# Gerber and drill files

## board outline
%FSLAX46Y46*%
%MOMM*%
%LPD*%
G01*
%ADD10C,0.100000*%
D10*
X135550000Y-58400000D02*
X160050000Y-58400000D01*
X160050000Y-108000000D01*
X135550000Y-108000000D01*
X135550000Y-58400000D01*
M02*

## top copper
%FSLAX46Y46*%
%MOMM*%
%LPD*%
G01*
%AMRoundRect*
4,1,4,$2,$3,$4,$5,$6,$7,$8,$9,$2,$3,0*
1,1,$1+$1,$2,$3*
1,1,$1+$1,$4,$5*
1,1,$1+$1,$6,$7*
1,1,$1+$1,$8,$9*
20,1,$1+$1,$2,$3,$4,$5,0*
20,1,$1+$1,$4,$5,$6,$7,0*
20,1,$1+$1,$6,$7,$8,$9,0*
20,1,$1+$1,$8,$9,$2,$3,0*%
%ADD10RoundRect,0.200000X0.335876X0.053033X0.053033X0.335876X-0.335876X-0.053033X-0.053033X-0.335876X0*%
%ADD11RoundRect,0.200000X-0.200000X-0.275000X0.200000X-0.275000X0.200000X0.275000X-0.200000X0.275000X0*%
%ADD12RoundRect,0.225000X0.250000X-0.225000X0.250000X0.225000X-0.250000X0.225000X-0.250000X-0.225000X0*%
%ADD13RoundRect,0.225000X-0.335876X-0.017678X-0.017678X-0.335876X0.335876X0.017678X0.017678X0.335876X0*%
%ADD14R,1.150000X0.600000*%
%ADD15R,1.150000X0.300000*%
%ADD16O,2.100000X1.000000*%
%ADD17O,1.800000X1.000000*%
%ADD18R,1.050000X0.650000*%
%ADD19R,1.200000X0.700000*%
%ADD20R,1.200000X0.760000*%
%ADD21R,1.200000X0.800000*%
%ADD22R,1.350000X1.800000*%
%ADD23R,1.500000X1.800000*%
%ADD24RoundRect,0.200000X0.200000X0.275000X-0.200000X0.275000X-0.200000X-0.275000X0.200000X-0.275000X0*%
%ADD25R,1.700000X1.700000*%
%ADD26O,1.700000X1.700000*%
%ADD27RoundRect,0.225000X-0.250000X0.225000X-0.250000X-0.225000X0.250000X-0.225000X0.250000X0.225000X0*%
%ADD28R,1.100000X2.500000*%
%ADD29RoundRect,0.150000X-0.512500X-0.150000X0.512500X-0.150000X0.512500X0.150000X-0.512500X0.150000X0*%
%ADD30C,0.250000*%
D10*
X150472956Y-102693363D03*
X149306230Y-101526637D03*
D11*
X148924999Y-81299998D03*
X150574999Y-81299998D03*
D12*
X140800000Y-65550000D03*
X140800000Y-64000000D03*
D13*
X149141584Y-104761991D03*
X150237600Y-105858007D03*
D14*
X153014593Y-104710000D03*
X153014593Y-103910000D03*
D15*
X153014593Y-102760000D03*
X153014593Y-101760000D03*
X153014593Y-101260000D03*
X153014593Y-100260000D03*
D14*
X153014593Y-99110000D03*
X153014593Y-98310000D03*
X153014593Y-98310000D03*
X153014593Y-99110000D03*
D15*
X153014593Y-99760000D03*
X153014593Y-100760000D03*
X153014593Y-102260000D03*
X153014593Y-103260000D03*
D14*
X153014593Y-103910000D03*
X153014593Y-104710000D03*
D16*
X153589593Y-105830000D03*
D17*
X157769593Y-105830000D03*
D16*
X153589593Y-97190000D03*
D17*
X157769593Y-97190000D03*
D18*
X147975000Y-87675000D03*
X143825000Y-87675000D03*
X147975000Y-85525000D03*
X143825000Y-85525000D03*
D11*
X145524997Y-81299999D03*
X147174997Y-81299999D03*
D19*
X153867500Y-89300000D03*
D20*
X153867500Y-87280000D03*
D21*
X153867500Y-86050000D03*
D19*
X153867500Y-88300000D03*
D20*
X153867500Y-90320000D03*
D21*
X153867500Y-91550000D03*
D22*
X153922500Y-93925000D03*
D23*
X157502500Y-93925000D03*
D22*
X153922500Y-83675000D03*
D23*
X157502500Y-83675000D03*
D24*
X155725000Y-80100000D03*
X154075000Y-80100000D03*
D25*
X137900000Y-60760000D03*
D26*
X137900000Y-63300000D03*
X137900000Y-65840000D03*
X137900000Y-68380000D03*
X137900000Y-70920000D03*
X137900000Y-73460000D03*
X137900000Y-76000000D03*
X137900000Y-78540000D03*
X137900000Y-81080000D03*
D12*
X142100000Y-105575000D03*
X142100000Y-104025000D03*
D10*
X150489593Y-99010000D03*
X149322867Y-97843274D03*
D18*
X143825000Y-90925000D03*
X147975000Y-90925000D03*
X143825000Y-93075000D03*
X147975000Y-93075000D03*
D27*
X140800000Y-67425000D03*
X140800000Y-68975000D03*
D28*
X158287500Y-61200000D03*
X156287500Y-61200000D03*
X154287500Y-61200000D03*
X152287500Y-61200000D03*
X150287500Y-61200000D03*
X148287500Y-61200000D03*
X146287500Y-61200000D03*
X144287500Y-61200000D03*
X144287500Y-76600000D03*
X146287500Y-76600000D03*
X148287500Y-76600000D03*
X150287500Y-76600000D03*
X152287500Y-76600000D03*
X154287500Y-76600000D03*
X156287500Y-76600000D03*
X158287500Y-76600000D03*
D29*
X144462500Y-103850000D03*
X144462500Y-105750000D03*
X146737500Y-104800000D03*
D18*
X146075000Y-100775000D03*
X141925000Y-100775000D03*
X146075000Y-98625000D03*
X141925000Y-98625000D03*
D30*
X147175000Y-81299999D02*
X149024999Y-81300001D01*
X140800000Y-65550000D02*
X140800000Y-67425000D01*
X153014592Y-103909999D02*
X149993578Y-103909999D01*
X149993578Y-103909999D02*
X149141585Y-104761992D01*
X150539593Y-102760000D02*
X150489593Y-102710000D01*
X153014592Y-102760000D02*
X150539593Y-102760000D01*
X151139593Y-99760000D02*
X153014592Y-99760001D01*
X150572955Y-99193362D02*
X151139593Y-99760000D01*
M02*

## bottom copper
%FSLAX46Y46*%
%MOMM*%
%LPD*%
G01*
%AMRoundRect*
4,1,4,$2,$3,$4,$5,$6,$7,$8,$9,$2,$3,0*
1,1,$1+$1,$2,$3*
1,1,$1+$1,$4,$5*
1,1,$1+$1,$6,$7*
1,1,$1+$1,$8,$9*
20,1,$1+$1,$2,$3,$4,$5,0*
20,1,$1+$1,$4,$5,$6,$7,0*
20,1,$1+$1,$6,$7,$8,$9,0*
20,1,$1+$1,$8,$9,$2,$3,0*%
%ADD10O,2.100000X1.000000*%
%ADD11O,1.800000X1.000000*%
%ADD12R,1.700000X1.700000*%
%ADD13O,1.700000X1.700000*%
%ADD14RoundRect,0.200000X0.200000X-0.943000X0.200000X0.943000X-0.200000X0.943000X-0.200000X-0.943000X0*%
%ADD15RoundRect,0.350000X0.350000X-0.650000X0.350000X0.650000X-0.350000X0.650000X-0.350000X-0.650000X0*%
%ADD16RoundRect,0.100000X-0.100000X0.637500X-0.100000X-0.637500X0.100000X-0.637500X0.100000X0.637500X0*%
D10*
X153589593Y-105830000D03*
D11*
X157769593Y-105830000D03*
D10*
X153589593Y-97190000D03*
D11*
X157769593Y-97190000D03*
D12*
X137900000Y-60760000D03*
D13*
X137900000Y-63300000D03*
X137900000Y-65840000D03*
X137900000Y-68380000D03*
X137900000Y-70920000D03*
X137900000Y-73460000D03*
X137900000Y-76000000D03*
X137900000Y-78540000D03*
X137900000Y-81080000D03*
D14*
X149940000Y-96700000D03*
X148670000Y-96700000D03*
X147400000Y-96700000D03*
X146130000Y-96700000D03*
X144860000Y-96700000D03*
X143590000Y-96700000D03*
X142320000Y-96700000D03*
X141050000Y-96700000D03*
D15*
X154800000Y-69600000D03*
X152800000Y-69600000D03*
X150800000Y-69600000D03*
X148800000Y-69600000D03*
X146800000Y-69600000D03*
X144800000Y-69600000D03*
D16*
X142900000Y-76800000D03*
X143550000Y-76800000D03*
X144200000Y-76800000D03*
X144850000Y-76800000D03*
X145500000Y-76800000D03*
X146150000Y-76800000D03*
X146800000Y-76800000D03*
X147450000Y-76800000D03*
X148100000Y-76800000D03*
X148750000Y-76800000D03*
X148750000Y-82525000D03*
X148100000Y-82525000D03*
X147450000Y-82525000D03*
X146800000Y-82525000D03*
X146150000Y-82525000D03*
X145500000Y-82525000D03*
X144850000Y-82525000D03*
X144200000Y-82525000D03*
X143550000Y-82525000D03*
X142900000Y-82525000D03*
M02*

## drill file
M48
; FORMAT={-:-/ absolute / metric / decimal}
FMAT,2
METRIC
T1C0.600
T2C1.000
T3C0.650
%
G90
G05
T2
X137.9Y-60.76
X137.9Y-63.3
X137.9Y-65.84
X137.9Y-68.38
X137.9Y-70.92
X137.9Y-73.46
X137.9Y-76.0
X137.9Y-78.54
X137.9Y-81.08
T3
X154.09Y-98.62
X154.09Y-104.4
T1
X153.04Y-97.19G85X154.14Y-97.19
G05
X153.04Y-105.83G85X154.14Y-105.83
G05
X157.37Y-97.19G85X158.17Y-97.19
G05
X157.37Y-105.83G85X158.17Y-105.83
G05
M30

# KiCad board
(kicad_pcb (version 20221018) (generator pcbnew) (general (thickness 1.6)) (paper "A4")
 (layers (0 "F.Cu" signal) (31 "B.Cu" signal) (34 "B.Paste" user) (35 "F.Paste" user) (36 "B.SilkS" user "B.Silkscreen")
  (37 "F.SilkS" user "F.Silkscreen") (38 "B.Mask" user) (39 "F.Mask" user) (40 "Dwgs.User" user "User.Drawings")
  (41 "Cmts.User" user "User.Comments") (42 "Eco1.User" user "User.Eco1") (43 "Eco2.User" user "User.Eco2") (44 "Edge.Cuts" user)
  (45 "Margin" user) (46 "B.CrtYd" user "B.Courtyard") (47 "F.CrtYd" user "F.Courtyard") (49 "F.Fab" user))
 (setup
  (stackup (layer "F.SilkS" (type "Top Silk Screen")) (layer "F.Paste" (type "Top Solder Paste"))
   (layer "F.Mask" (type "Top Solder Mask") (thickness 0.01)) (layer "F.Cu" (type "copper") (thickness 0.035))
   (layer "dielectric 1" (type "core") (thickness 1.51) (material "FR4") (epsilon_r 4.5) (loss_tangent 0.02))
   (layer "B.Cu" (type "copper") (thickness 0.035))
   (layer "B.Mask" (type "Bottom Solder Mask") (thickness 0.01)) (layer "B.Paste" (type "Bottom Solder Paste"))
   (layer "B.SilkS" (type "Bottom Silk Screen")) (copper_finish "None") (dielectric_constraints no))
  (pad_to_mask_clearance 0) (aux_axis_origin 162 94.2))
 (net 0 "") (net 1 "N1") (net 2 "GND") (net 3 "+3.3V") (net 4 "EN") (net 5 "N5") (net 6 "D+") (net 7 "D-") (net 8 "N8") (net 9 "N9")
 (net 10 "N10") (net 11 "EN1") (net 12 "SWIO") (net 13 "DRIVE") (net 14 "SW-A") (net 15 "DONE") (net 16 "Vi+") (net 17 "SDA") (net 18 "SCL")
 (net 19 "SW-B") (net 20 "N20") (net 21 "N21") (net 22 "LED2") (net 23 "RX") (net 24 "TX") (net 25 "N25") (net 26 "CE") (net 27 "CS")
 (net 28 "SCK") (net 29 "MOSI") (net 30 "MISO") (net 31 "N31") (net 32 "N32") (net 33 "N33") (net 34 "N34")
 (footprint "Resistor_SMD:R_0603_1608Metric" (layer "F.Cu") (at 149.889593 102.11 135)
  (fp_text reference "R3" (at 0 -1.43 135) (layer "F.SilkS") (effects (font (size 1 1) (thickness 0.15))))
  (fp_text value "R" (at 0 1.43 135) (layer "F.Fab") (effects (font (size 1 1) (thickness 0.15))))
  (pad "1" smd roundrect (at -0.825 0 135) (size 0.8 0.95) (layers "F.Cu" "F.Paste" "F.Mask") (roundrect_rratio 0.25) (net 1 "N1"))
  (pad "2" smd roundrect (at 0.825 0 135) (size 0.8 0.95) (layers "F.Cu" "F.Paste" "F.Mask") (roundrect_rratio 0.25) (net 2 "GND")))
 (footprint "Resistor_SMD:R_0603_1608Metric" (layer "F.Cu") (at 149.749999 81.299998)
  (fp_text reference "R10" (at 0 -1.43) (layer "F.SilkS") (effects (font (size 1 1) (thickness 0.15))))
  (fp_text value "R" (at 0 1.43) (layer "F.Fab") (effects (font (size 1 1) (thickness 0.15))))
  (pad "1" smd roundrect (at -0.825 0) (size 0.8 0.95) (layers "F.Cu" "F.Paste" "F.Mask") (roundrect_rratio 0.25) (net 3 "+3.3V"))
  (pad "2" smd roundrect (at 0.825 0) (size 0.8 0.95) (layers "F.Cu" "F.Paste" "F.Mask") (roundrect_rratio 0.25) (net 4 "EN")))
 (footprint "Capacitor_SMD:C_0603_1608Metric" (layer "F.Cu") (at 140.8 64.775 90)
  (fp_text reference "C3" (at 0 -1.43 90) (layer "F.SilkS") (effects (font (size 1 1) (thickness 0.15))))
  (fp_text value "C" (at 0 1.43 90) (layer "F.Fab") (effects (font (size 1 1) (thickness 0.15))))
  (pad "1" smd roundrect (at -0.775 0 90) (size 0.9 0.95) (layers "F.Cu" "F.Paste" "F.Mask") (roundrect_rratio 0.25) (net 3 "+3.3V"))
  (pad "2" smd roundrect (at 0.775 0 90) (size 0.9 0.95) (layers "F.Cu" "F.Paste" "F.Mask") (roundrect_rratio 0.25) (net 2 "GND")))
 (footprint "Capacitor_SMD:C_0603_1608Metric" (layer "F.Cu") (at 149.689592 105.309999 -45)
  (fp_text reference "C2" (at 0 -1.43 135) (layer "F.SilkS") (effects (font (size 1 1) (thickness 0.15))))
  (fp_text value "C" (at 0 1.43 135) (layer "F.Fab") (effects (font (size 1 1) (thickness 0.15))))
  (pad "1" smd roundrect (at -0.775 0 315) (size 0.9 0.95) (layers "F.Cu" "F.Paste" "F.Mask") (roundrect_rratio 0.25) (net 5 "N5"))
  (pad "2" smd roundrect (at 0.775 0 315) (size 0.9 0.95) (layers "F.Cu" "F.Paste" "F.Mask") (roundrect_rratio 0.25) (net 2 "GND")))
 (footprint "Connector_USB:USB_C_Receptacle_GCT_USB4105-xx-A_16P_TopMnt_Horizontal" (layer "F.Cu") (at 156.694593 101.51 90)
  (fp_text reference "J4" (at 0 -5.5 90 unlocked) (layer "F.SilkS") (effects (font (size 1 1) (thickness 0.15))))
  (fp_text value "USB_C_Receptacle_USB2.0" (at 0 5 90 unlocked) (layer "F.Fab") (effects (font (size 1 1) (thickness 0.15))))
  (pad "" np_thru_hole circle (at -2.89 -2.605 90) (size 0.65 0.65) (drill 0.65) (layers "F&B.Cu" "*.Mask"))
  (pad "" np_thru_hole circle (at 2.89 -2.605 90) (size 0.65 0.65) (drill 0.65) (layers "F&B.Cu" "*.Mask"))
  (pad "A1" smd rect (at -3.2 -3.68 90) (size 0.6 1.15) (layers "F.Cu" "F.Paste" "F.Mask") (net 2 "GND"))
  (pad "A4" smd rect (at -2.4 -3.68 90) (size 0.6 1.15) (layers "F.Cu" "F.Paste" "F.Mask") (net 5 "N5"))
  (pad "A5" smd rect (at -1.25 -3.68 90) (size 0.3 1.15) (layers "F.Cu" "F.Paste" "F.Mask") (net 1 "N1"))
  (pad "A6" smd rect (at -0.25 -3.68 90) (size 0.3 1.15) (layers "F.Cu" "F.Paste" "F.Mask") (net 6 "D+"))
  (pad "A7" smd rect (at 0.25 -3.68 90) (size 0.3 1.15) (layers "F.Cu" "F.Paste" "F.Mask") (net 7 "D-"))
  (pad "A8" smd rect (at 1.25 -3.68 90) (size 0.3 1.15) (layers "F.Cu" "F.Paste" "F.Mask") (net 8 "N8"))
  (pad "A9" smd rect (at 2.4 -3.68 90) (size 0.6 1.15) (layers "F.Cu" "F.Paste" "F.Mask") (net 5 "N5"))
  (pad "A12" smd rect (at 3.2 -3.68 90) (size 0.6 1.15) (layers "F.Cu" "F.Paste" "F.Mask") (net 2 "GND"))
  (pad "B1" smd rect (at 3.2 -3.68 90) (size 0.6 1.15) (layers "F.Cu" "F.Paste" "F.Mask") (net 2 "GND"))
  (pad "B4" smd rect (at 2.4 -3.68 90) (size 0.6 1.15) (layers "F.Cu" "F.Paste" "F.Mask") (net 5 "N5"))
  (pad "B5" smd rect (at 1.75 -3.68 90) (size 0.3 1.15) (layers "F.Cu" "F.Paste" "F.Mask") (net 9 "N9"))
  (pad "B6" smd rect (at 0.75 -3.68 90) (size 0.3 1.15) (layers "F.Cu" "F.Paste" "F.Mask") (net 6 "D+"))
  (pad "B7" smd rect (at -0.75 -3.68 90) (size 0.3 1.15) (layers "F.Cu" "F.Paste" "F.Mask") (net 7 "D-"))
  (pad "B8" smd rect (at -1.75 -3.68 90) (size 0.3 1.15) (layers "F.Cu" "F.Paste" "F.Mask") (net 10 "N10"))
  (pad "B9" smd rect (at -2.4 -3.68 90) (size 0.6 1.15) (layers "F.Cu" "F.Paste" "F.Mask") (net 5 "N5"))
  (pad "B12" smd rect (at -3.2 -3.68 90) (size 0.6 1.15) (layers "F.Cu" "F.Paste" "F.Mask") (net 2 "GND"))
  (pad "S1" thru_hole oval (at -4.32 -3.105 90) (size 1 2.1) (drill oval 0.6 1.7) (layers "*.Cu" "*.Mask" "F.Paste") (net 2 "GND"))
  (pad "S1" thru_hole oval (at -4.32 1.075 90) (size 1 1.8) (drill oval 0.6 1.4) (layers "*.Cu" "*.Mask" "F.Paste") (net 2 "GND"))
  (pad "S1" thru_hole oval (at 4.32 -3.105 90) (size 1 2.1) (drill oval 0.6 1.7) (layers "*.Cu" "*.Mask" "F.Paste") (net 2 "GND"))
  (pad "S1" thru_hole oval (at 4.32 1.075 90) (size 1 1.8) (drill oval 0.6 1.4) (layers "*.Cu" "*.Mask" "F.Paste") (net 2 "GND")))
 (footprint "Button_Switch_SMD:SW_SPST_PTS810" (layer "F.Cu") (at 145.9 86.6 180)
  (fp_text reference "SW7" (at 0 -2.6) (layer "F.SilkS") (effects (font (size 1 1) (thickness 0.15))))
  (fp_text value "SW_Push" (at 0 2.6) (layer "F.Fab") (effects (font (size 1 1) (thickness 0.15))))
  (pad "1" smd rect (at -2.075 -1.075 180) (size 1.05 0.65) (layers "F.Cu" "F.Paste" "F.Mask") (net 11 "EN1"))
  (pad "1" smd rect (at 2.075 -1.075 180) (size 1.05 0.65) (layers "F.Cu" "F.Paste" "F.Mask") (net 11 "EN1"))
  (pad "2" smd rect (at -2.075 1.075 180) (size 1.05 0.65) (layers "F.Cu" "F.Paste" "F.Mask") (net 2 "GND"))
  (pad "2" smd rect (at 2.075 1.075 180) (size 1.05 0.65) (layers "F.Cu" "F.Paste" "F.Mask") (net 2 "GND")))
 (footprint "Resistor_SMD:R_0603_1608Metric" (layer "F.Cu") (at 146.349997 81.299999)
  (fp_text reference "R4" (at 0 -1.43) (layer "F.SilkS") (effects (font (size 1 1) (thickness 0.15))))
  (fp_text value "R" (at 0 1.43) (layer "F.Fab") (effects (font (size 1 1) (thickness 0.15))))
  (pad "1" smd roundrect (at -0.825 0) (size 0.8 0.95) (layers "F.Cu" "F.Paste" "F.Mask") (roundrect_rratio 0.25) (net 11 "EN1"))
  (pad "2" smd roundrect (at 0.825 0) (size 0.8 0.95) (layers "F.Cu" "F.Paste" "F.Mask") (roundrect_rratio 0.25) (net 3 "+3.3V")))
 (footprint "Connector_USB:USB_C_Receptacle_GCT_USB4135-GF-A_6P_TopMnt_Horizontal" (layer "F.Cu") (at 156.9 88.8 90)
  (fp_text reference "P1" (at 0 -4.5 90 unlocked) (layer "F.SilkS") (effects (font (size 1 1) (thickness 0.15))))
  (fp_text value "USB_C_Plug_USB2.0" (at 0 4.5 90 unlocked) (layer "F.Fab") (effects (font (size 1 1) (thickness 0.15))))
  (pad "A5" smd rect (at -0.5 -3.0325 90) (size 0.7 1.2) (layers "F.Cu" "F.Paste" "F.Mask") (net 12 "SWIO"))
  (pad "A9" smd rect (at 1.52 -3.0325 270) (size 0.76 1.2) (layers "F.Cu" "F.Paste" "F.Mask") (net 3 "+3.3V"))
  (pad "A12" smd rect (at 2.75 -3.0325 270) (size 0.8 1.2) (layers "F.Cu" "F.Paste" "F.Mask") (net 2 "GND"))
  (pad "B5" smd rect (at 0.5 -3.0325 270) (size 0.7 1.2) (layers "F.Cu" "F.Paste" "F.Mask") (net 12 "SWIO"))
  (pad "B9" smd rect (at -1.52 -3.0325 90) (size 0.76 1.2) (layers "F.Cu" "F.Paste" "F.Mask") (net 3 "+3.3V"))
  (pad "B12" smd rect (at -2.75 -3.0325 90) (size 0.8 1.2) (layers "F.Cu" "F.Paste" "F.Mask") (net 2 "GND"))
  (pad "S1" smd rect (at -5.125 -2.9775 90) (size 1.8 1.35) (layers "F.Cu" "F.Paste" "F.Mask") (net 2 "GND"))
  (pad "S1" smd rect (at -5.125 0.6025 90) (size 1.8 1.5) (layers "F.Cu" "F.Paste" "F.Mask") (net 2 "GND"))
  (pad "S1" smd rect (at 5.125 -2.9775 90) (size 1.8 1.35) (layers "F.Cu" "F.Paste" "F.Mask") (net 2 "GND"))
  (pad "S1" smd rect (at 5.125 0.6025 90) (size 1.8 1.5) (layers "F.Cu" "F.Paste" "F.Mask") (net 2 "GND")))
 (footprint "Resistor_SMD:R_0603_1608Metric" (layer "F.Cu") (at 154.9 80.1 180)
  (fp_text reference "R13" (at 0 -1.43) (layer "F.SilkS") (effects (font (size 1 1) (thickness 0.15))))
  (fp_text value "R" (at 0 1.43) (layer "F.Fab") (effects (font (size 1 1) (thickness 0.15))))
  (pad "1" smd roundrect (at -0.825 0 180) (size 0.8 0.95) (layers "F.Cu" "F.Paste" "F.Mask") (roundrect_rratio 0.25) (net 2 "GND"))
  (pad "2" smd roundrect (at 0.825 0 180) (size 0.8 0.95) (layers "F.Cu" "F.Paste" "F.Mask") (roundrect_rratio 0.25) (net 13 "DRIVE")))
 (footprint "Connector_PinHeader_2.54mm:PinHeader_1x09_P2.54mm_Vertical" (layer "F.Cu") (at 137.9 60.76)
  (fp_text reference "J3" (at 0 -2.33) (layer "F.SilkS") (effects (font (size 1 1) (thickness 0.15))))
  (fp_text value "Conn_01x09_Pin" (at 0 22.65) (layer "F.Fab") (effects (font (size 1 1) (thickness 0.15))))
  (pad "1" thru_hole rect (at 0 0) (size 1.7 1.7) (drill 1) (layers "*.Cu" "*.Mask") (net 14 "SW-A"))
  (pad "2" thru_hole oval (at 0 2.54) (size 1.7 1.7) (drill 1) (layers "*.Cu" "*.Mask") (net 2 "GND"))
  (pad "3" thru_hole oval (at 0 5.08) (size 1.7 1.7) (drill 1) (layers "*.Cu" "*.Mask") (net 3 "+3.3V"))
  (pad "4" thru_hole oval (at 0 7.62) (size 1.7 1.7) (drill 1) (layers "*.Cu" "*.Mask") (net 13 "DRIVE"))
  (pad "5" thru_hole oval (at 0 10.16) (size 1.7 1.7) (drill 1) (layers "*.Cu" "*.Mask") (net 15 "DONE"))
  (pad "6" thru_hole oval (at 0 12.7) (size 1.7 1.7) (drill 1) (layers "*.Cu" "*.Mask") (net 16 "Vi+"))
  (pad "7" thru_hole oval (at 0 15.24) (size 1.7 1.7) (drill 1) (layers "*.Cu" "*.Mask") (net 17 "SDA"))
  (pad "8" thru_hole oval (at 0 17.78) (size 1.7 1.7) (drill 1) (layers "*.Cu" "*.Mask") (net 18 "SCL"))
  (pad "9" thru_hole oval (at 0 20.32) (size 1.7 1.7) (drill 1) (layers "*.Cu" "*.Mask") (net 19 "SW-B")))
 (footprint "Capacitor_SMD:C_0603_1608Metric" (layer "F.Cu") (at 142.1 104.8 90)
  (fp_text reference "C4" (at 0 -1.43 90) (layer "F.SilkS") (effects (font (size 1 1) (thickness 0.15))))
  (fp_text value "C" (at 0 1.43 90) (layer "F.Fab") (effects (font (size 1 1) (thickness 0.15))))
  (pad "1" smd roundrect (at -0.775 0 90) (size 0.9 0.95) (layers "F.Cu" "F.Paste" "F.Mask") (roundrect_rratio 0.25) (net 3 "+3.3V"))
  (pad "2" smd roundrect (at 0.775 0 90) (size 0.9 0.95) (layers "F.Cu" "F.Paste" "F.Mask") (roundrect_rratio 0.25) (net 2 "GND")))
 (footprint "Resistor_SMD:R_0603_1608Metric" (layer "F.Cu") (at 149.90623 98.426637 135)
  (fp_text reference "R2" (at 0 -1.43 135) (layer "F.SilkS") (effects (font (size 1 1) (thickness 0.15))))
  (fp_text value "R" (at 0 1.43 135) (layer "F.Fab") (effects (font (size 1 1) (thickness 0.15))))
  (pad "1" smd roundrect (at -0.825 0 135) (size 0.8 0.95) (layers "F.Cu" "F.Paste" "F.Mask") (roundrect_rratio 0.25) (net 9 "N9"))
  (pad "2" smd roundrect (at 0.825 0 135) (size 0.8 0.95) (layers "F.Cu" "F.Paste" "F.Mask") (roundrect_rratio 0.25) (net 2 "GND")))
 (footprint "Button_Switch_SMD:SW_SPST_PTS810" (layer "F.Cu") (at 145.9 92)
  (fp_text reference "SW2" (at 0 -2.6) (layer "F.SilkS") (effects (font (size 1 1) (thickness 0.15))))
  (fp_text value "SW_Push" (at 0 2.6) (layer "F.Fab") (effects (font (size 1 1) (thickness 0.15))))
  (pad "1" smd rect (at -2.075 -1.075) (size 1.05 0.65) (layers "F.Cu" "F.Paste" "F.Mask") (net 2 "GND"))
  (pad "1" smd rect (at 2.075 -1.075) (size 1.05 0.65) (layers "F.Cu" "F.Paste" "F.Mask") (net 2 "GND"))
  (pad "2" smd rect (at -2.075 1.075) (size 1.05 0.65) (layers "F.Cu" "F.Paste" "F.Mask") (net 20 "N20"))
  (pad "2" smd rect (at 2.075 1.075) (size 1.05 0.65) (layers "F.Cu" "F.Paste" "F.Mask") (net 20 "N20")))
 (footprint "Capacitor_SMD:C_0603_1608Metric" (layer "F.Cu") (at 140.8 68.2 -90)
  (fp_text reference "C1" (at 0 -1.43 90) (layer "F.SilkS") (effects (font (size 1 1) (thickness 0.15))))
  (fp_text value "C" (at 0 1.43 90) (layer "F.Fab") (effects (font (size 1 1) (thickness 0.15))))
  (pad "1" smd roundrect (at -0.775 0 270) (size 0.9 0.95) (layers "F.Cu" "F.Paste" "F.Mask") (roundrect_rratio 0.25) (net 3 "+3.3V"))
  (pad "2" smd roundrect (at 0.775 0 270) (size 0.9 0.95) (layers "F.Cu" "F.Paste" "F.Mask") (roundrect_rratio 0.25) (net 2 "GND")))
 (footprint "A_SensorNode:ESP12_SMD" (layer "F.Cu") (at 160.8875 60.85 -90)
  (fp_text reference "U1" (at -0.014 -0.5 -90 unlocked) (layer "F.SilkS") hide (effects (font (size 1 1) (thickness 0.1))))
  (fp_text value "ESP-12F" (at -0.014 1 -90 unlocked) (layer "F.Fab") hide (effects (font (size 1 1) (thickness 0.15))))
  (pad "1" smd rect (at 1.05 2.6 270) (size 2.5 1.1) (drill (offset -0.7 0)) (layers "F.Cu" "F.Paste" "F.Mask") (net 11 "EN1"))
  (pad "2" smd rect (at 1.05 4.6 270) (size 2.5 1.1) (drill (offset -0.7 0)) (layers "F.Cu" "F.Paste" "F.Mask") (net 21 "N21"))
  (pad "3" smd rect (at 1.05 6.6 270) (size 2.5 1.1) (drill (offset -0.7 0)) (layers "F.Cu" "F.Paste" "F.Mask") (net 4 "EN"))
  (pad "4" smd rect (at 1.05 8.6 270) (size 2.5 1.1) (drill (offset -0.7 0)) (layers "F.Cu" "F.Paste" "F.Mask") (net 11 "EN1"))
  (pad "5" smd rect (at 1.05 10.6 270) (size 2.5 1.1) (drill (offset -0.7 0)) (layers "F.Cu" "F.Paste" "F.Mask") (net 14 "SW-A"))
  (pad "6" smd rect (at 1.05 12.6 270) (size 2.5 1.1) (drill (offset -0.7 0)) (layers "F.Cu" "F.Paste" "F.Mask") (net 19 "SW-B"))
  (pad "7" smd rect (at 1.05 14.6 270) (size 2.5 1.1) (drill (offset -0.7 0)) (layers "F.Cu" "F.Paste" "F.Mask") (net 15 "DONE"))
  (pad "8" smd rect (at 1.05 16.6 270) (size 2.5 1.1) (drill (offset -0.7 0)) (layers "F.Cu" "F.Paste" "F.Mask") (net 3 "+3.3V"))
  (pad "9" smd rect (at 15.05 16.6 270) (size 2.5 1.1) (drill (offset 0.7 0)) (layers "F.Cu" "F.Paste" "F.Mask") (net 2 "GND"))
  (pad "10" smd rect (at 15.05 14.6 270) (size 2.5 1.1) (drill (offset 0.7 0)) (layers "F.Cu" "F.Paste" "F.Mask") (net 13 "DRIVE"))
  (pad "11" smd rect (at 15.05 12.6 270) (size 2.5 1.1) (drill (offset 0.7 0)) (layers "F.Cu" "F.Paste" "F.Mask") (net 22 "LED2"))
  (pad "12" smd rect (at 15.05 10.6 270) (size 2.5 1.1) (drill (offset 0.7 0)) (layers "F.Cu" "F.Paste" "F.Mask") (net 20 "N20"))
  (pad "13" smd rect (at 15.05 8.6 270) (size 2.5 1.1) (drill (offset 0.7 0)) (layers "F.Cu" "F.Paste" "F.Mask") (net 17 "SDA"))
  (pad "14" smd rect (at 15.05 6.6 270) (size 2.5 1.1) (drill (offset 0.7 0)) (layers "F.Cu" "F.Paste" "F.Mask") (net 18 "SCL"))
  (pad "15" smd rect (at 15.05 4.6 270) (size 2.5 1.1) (drill (offset 0.7 0)) (layers "F.Cu" "F.Paste" "F.Mask") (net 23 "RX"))
  (pad "16" smd rect (at 15.05 2.6 270) (size 2.5 1.1) (drill (offset 0.7 0)) (layers "F.Cu" "F.Paste" "F.Mask") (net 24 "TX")))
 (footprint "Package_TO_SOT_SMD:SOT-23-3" (layer "F.Cu") (at 145.6 104.8)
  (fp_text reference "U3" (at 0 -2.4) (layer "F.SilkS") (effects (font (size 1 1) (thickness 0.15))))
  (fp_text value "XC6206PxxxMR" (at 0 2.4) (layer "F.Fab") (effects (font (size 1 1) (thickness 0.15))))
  (pad "1" smd roundrect (at -1.1375 -0.95) (size 1.325 0.6) (layers "F.Cu" "F.Paste" "F.Mask") (roundrect_rratio 0.25) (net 2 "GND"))
  (pad "2" smd roundrect (at -1.1375 0.95) (size 1.325 0.6) (layers "F.Cu" "F.Paste" "F.Mask") (roundrect_rratio 0.25) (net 3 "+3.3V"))
  (pad "3" smd roundrect (at 1.1375 0) (size 1.325 0.6) (layers "F.Cu" "F.Paste" "F.Mask") (roundrect_rratio 0.25) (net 5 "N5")))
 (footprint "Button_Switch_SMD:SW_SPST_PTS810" (layer "F.Cu") (at 144 99.7 180)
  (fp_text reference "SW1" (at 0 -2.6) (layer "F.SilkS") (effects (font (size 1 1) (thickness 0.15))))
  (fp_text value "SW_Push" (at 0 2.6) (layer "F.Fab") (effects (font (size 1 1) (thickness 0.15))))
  (pad "1" smd rect (at -2.075 -1.075 180) (size 1.05 0.65) (layers "F.Cu" "F.Paste" "F.Mask") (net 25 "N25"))
  (pad "1" smd rect (at 2.075 -1.075 180) (size 1.05 0.65) (layers "F.Cu" "F.Paste" "F.Mask") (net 25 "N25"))
  (pad "2" smd rect (at -2.075 1.075 180) (size 1.05 0.65) (layers "F.Cu" "F.Paste" "F.Mask") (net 2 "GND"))
  (pad "2" smd rect (at 2.075 1.075 180) (size 1.05 0.65) (layers "F.Cu" "F.Paste" "F.Mask") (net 2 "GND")))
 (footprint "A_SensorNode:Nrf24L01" (layer "B.Cu") (at 149.94 96.7 90)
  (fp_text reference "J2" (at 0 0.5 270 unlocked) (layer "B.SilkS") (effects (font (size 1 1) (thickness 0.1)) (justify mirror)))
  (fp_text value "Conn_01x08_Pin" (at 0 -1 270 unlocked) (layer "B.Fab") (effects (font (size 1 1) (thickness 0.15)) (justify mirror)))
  (pad "1" smd roundrect (at 0 0 90) (size 2.286 0.8) (layers "B.Cu" "B.Paste" "B.Mask") (roundrect_rratio 0.25) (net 3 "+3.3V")
   (thermal_bridge_angle 45))
  (pad "2" smd roundrect (at 0 -1.27 90) (size 2.286 0.8) (layers "B.Cu" "B.Paste" "B.Mask") (roundrect_rratio 0.25) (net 2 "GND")
   (thermal_bridge_angle 45))
  (pad "3" smd roundrect (at 0 -2.54 90) (size 2.286 0.8) (layers "B.Cu" "B.Paste" "B.Mask") (roundrect_rratio 0.25) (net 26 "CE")
   (thermal_bridge_angle 45))
  (pad "4" smd roundrect (at 0 -3.81 90) (size 2.286 0.8) (layers "B.Cu" "B.Paste" "B.Mask") (roundrect_rratio 0.25) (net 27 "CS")
   (thermal_bridge_angle 45))
  (pad "5" smd roundrect (at 0 -5.08 90) (size 2.286 0.8) (layers "B.Cu" "B.Paste" "B.Mask") (roundrect_rratio 0.25) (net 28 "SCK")
   (thermal_bridge_angle 45))
  (pad "6" smd roundrect (at 0 -6.35 90) (size 2.286 0.8) (layers "B.Cu" "B.Paste" "B.Mask") (roundrect_rratio 0.25) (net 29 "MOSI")
   (thermal_bridge_angle 45))
  (pad "7" smd roundrect (at 0 -7.62 90) (size 2.286 0.8) (layers "B.Cu" "B.Paste" "B.Mask") (roundrect_rratio 0.25) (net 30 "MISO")
   (thermal_bridge_angle 45))
  (pad "8" smd roundrect (at 0 -8.89 90) (size 2.286 0.8) (layers "B.Cu" "B.Paste" "B.Mask") (roundrect_rratio 0.25) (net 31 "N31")
   (thermal_bridge_angle 45)))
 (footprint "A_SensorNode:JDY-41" (layer "B.Cu") (at 156.8 47.7 180)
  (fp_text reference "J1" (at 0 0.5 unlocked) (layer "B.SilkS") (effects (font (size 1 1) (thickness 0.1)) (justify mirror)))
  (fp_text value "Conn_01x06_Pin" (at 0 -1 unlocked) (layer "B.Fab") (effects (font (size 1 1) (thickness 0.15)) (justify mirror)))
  (pad "1" smd roundrect (at 2 -21.9 90) (size 2 1.4) (layers "B.Cu" "B.Paste" "B.Mask") (roundrect_rratio 0.25) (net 3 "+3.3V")
   (thermal_bridge_angle 45))
  (pad "2" smd roundrect (at 4 -21.9 90) (size 2 1.4) (layers "B.Cu" "B.Paste" "B.Mask") (roundrect_rratio 0.25) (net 23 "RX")
   (thermal_bridge_angle 45))
  (pad "3" smd roundrect (at 6 -21.9 90) (size 2 1.4) (layers "B.Cu" "B.Paste" "B.Mask") (roundrect_rratio 0.25) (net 24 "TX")
   (thermal_bridge_angle 45))
  (pad "4" smd roundrect (at 8 -21.9 90) (size 2 1.4) (layers "B.Cu" "B.Paste" "B.Mask") (roundrect_rratio 0.25) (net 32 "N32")
   (thermal_bridge_angle 45))
  (pad "5" smd roundrect (at 10 -21.9 90) (size 2 1.4) (layers "B.Cu" "B.Paste" "B.Mask") (roundrect_rratio 0.25) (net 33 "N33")
   (thermal_bridge_angle 45))
  (pad "6" smd roundrect (at 12 -21.9 90) (size 2 1.4) (layers "B.Cu" "B.Paste" "B.Mask") (roundrect_rratio 0.25) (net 2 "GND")
   (thermal_bridge_angle 45)))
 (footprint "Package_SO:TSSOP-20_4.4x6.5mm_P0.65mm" (layer "B.Cu") (at 145.825 79.6625 -90)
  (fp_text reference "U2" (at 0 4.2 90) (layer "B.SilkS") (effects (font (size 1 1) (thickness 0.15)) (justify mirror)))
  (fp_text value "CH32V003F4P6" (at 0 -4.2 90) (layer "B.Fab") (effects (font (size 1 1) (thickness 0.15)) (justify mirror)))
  (pad "1" smd roundrect (at -2.8625 2.925 270) (size 1.475 0.4) (layers "B.Cu" "B.Paste" "B.Mask") (roundrect_rratio 0.25) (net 7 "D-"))
  (pad "2" smd roundrect (at -2.8625 2.275 270) (size 1.475 0.4) (layers "B.Cu" "B.Paste" "B.Mask") (roundrect_rratio 0.25) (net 23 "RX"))
  (pad "3" smd roundrect (at -2.8625 1.625 270) (size 1.475 0.4) (layers "B.Cu" "B.Paste" "B.Mask") (roundrect_rratio 0.25) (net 24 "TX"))
  (pad "4" smd roundrect (at -2.8625 0.975 270) (size 1.475 0.4) (layers "B.Cu" "B.Paste" "B.Mask") (roundrect_rratio 0.25) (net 25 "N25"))
  (pad "5" smd roundrect (at -2.8625 0.325 270) (size 1.475 0.4) (layers "B.Cu" "B.Paste" "B.Mask") (roundrect_rratio 0.25) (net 14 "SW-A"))
  (pad "6" smd roundrect (at -2.8625 -0.325 270) (size 1.475 0.4) (layers "B.Cu" "B.Paste" "B.Mask") (roundrect_rratio 0.25) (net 19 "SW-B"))
  (pad "7" smd roundrect (at -2.8625 -0.975 270) (size 1.475 0.4) (layers "B.Cu" "B.Paste" "B.Mask") (roundrect_rratio 0.25) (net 2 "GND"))
  (pad "8" smd roundrect (at -2.8625 -1.625 270) (size 1.475 0.4) (layers "B.Cu" "B.Paste" "B.Mask") (roundrect_rratio 0.25)
   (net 13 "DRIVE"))
  (pad "9" smd roundrect (at -2.8625 -2.275 270) (size 1.475 0.4) (layers "B.Cu" "B.Paste" "B.Mask") (roundrect_rratio 0.25) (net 3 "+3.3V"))
  (pad "10" smd roundrect (at -2.8625 -2.925 270) (size 1.475 0.4) (layers "B.Cu" "B.Paste" "B.Mask") (roundrect_rratio 0.25) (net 27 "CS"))
  (pad "11" smd roundrect (at 2.8625 -2.925 270) (size 1.475 0.4) (layers "B.Cu" "B.Paste" "B.Mask") (roundrect_rratio 0.25) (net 17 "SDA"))
  (pad "12" smd roundrect (at 2.8625 -2.275 270) (size 1.475 0.4) (layers "B.Cu" "B.Paste" "B.Mask") (roundrect_rratio 0.25) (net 18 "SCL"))
  (pad "13" smd roundrect (at 2.8625 -1.625 270) (size 1.475 0.4) (layers "B.Cu" "B.Paste" "B.Mask") (roundrect_rratio 0.25) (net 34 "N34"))
  (pad "14" smd roundrect (at 2.8625 -0.975 270) (size 1.475 0.4) (layers "B.Cu" "B.Paste" "B.Mask") (roundrect_rratio 0.25) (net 26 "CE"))
  (pad "15" smd roundrect (at 2.8625 -0.325 270) (size 1.475 0.4) (layers "B.Cu" "B.Paste" "B.Mask") (roundrect_rratio 0.25) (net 28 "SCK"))
  (pad "16" smd roundrect (at 2.8625 0.325 270) (size 1.475 0.4) (layers "B.Cu" "B.Paste" "B.Mask") (roundrect_rratio 0.25) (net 29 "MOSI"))
  (pad "17" smd roundrect (at 2.8625 0.975 270) (size 1.475 0.4) (layers "B.Cu" "B.Paste" "B.Mask") (roundrect_rratio 0.25) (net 30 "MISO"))
  (pad "18" smd roundrect (at 2.8625 1.625 270) (size 1.475 0.4) (layers "B.Cu" "B.Paste" "B.Mask") (roundrect_rratio 0.25) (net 12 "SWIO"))
  (pad "19" smd roundrect (at 2.8625 2.275 270) (size 1.475 0.4) (layers "B.Cu" "B.Paste" "B.Mask") (roundrect_rratio 0.25) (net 15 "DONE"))
  (pad "20" smd roundrect (at 2.8625 2.925 270) (size 1.475 0.4) (layers "B.Cu" "B.Paste" "B.Mask") (roundrect_rratio 0.25) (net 6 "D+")))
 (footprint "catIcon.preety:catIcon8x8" (layer "B.Cu") (at 125.1 63.8 180)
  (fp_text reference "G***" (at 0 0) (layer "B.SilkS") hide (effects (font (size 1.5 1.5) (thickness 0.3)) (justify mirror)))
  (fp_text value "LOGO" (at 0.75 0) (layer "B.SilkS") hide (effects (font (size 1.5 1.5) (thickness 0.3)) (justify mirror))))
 (gr_rect (start 135.55 58.4) (end 160.05 108) (stroke (width 0.1) (type default)) (fill none) (layer "Edge.Cuts"))
 (segment (start 147.175 81.299999) (end 149.024999 81.300001) (width 0.25) (layer "F.Cu") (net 3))
 (segment (start 140.8 65.55) (end 140.8 67.425) (width 0.25) (layer "F.Cu") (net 3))
 (segment (start 153.014592 103.909999) (end 149.993578 103.909999) (width 0.25) (layer "F.Cu") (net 5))
 (segment (start 149.993578 103.909999) (end 149.141585 104.761992) (width 0.25) (layer "F.Cu") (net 5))
 (segment (start 150.539593 102.76) (end 150.489593 102.71) (width 0.25) (layer "F.Cu") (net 1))
 (segment (start 153.014592 102.76) (end 150.539593 102.76) (width 0.25) (layer "F.Cu") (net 1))
 (segment (start 151.139593 99.76) (end 153.014592 99.760001) (width 0.25) (layer "F.Cu") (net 9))
 (segment (start 150.572955 99.193362) (end 151.139593 99.76) (width 0.25) (layer "F.Cu") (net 9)))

